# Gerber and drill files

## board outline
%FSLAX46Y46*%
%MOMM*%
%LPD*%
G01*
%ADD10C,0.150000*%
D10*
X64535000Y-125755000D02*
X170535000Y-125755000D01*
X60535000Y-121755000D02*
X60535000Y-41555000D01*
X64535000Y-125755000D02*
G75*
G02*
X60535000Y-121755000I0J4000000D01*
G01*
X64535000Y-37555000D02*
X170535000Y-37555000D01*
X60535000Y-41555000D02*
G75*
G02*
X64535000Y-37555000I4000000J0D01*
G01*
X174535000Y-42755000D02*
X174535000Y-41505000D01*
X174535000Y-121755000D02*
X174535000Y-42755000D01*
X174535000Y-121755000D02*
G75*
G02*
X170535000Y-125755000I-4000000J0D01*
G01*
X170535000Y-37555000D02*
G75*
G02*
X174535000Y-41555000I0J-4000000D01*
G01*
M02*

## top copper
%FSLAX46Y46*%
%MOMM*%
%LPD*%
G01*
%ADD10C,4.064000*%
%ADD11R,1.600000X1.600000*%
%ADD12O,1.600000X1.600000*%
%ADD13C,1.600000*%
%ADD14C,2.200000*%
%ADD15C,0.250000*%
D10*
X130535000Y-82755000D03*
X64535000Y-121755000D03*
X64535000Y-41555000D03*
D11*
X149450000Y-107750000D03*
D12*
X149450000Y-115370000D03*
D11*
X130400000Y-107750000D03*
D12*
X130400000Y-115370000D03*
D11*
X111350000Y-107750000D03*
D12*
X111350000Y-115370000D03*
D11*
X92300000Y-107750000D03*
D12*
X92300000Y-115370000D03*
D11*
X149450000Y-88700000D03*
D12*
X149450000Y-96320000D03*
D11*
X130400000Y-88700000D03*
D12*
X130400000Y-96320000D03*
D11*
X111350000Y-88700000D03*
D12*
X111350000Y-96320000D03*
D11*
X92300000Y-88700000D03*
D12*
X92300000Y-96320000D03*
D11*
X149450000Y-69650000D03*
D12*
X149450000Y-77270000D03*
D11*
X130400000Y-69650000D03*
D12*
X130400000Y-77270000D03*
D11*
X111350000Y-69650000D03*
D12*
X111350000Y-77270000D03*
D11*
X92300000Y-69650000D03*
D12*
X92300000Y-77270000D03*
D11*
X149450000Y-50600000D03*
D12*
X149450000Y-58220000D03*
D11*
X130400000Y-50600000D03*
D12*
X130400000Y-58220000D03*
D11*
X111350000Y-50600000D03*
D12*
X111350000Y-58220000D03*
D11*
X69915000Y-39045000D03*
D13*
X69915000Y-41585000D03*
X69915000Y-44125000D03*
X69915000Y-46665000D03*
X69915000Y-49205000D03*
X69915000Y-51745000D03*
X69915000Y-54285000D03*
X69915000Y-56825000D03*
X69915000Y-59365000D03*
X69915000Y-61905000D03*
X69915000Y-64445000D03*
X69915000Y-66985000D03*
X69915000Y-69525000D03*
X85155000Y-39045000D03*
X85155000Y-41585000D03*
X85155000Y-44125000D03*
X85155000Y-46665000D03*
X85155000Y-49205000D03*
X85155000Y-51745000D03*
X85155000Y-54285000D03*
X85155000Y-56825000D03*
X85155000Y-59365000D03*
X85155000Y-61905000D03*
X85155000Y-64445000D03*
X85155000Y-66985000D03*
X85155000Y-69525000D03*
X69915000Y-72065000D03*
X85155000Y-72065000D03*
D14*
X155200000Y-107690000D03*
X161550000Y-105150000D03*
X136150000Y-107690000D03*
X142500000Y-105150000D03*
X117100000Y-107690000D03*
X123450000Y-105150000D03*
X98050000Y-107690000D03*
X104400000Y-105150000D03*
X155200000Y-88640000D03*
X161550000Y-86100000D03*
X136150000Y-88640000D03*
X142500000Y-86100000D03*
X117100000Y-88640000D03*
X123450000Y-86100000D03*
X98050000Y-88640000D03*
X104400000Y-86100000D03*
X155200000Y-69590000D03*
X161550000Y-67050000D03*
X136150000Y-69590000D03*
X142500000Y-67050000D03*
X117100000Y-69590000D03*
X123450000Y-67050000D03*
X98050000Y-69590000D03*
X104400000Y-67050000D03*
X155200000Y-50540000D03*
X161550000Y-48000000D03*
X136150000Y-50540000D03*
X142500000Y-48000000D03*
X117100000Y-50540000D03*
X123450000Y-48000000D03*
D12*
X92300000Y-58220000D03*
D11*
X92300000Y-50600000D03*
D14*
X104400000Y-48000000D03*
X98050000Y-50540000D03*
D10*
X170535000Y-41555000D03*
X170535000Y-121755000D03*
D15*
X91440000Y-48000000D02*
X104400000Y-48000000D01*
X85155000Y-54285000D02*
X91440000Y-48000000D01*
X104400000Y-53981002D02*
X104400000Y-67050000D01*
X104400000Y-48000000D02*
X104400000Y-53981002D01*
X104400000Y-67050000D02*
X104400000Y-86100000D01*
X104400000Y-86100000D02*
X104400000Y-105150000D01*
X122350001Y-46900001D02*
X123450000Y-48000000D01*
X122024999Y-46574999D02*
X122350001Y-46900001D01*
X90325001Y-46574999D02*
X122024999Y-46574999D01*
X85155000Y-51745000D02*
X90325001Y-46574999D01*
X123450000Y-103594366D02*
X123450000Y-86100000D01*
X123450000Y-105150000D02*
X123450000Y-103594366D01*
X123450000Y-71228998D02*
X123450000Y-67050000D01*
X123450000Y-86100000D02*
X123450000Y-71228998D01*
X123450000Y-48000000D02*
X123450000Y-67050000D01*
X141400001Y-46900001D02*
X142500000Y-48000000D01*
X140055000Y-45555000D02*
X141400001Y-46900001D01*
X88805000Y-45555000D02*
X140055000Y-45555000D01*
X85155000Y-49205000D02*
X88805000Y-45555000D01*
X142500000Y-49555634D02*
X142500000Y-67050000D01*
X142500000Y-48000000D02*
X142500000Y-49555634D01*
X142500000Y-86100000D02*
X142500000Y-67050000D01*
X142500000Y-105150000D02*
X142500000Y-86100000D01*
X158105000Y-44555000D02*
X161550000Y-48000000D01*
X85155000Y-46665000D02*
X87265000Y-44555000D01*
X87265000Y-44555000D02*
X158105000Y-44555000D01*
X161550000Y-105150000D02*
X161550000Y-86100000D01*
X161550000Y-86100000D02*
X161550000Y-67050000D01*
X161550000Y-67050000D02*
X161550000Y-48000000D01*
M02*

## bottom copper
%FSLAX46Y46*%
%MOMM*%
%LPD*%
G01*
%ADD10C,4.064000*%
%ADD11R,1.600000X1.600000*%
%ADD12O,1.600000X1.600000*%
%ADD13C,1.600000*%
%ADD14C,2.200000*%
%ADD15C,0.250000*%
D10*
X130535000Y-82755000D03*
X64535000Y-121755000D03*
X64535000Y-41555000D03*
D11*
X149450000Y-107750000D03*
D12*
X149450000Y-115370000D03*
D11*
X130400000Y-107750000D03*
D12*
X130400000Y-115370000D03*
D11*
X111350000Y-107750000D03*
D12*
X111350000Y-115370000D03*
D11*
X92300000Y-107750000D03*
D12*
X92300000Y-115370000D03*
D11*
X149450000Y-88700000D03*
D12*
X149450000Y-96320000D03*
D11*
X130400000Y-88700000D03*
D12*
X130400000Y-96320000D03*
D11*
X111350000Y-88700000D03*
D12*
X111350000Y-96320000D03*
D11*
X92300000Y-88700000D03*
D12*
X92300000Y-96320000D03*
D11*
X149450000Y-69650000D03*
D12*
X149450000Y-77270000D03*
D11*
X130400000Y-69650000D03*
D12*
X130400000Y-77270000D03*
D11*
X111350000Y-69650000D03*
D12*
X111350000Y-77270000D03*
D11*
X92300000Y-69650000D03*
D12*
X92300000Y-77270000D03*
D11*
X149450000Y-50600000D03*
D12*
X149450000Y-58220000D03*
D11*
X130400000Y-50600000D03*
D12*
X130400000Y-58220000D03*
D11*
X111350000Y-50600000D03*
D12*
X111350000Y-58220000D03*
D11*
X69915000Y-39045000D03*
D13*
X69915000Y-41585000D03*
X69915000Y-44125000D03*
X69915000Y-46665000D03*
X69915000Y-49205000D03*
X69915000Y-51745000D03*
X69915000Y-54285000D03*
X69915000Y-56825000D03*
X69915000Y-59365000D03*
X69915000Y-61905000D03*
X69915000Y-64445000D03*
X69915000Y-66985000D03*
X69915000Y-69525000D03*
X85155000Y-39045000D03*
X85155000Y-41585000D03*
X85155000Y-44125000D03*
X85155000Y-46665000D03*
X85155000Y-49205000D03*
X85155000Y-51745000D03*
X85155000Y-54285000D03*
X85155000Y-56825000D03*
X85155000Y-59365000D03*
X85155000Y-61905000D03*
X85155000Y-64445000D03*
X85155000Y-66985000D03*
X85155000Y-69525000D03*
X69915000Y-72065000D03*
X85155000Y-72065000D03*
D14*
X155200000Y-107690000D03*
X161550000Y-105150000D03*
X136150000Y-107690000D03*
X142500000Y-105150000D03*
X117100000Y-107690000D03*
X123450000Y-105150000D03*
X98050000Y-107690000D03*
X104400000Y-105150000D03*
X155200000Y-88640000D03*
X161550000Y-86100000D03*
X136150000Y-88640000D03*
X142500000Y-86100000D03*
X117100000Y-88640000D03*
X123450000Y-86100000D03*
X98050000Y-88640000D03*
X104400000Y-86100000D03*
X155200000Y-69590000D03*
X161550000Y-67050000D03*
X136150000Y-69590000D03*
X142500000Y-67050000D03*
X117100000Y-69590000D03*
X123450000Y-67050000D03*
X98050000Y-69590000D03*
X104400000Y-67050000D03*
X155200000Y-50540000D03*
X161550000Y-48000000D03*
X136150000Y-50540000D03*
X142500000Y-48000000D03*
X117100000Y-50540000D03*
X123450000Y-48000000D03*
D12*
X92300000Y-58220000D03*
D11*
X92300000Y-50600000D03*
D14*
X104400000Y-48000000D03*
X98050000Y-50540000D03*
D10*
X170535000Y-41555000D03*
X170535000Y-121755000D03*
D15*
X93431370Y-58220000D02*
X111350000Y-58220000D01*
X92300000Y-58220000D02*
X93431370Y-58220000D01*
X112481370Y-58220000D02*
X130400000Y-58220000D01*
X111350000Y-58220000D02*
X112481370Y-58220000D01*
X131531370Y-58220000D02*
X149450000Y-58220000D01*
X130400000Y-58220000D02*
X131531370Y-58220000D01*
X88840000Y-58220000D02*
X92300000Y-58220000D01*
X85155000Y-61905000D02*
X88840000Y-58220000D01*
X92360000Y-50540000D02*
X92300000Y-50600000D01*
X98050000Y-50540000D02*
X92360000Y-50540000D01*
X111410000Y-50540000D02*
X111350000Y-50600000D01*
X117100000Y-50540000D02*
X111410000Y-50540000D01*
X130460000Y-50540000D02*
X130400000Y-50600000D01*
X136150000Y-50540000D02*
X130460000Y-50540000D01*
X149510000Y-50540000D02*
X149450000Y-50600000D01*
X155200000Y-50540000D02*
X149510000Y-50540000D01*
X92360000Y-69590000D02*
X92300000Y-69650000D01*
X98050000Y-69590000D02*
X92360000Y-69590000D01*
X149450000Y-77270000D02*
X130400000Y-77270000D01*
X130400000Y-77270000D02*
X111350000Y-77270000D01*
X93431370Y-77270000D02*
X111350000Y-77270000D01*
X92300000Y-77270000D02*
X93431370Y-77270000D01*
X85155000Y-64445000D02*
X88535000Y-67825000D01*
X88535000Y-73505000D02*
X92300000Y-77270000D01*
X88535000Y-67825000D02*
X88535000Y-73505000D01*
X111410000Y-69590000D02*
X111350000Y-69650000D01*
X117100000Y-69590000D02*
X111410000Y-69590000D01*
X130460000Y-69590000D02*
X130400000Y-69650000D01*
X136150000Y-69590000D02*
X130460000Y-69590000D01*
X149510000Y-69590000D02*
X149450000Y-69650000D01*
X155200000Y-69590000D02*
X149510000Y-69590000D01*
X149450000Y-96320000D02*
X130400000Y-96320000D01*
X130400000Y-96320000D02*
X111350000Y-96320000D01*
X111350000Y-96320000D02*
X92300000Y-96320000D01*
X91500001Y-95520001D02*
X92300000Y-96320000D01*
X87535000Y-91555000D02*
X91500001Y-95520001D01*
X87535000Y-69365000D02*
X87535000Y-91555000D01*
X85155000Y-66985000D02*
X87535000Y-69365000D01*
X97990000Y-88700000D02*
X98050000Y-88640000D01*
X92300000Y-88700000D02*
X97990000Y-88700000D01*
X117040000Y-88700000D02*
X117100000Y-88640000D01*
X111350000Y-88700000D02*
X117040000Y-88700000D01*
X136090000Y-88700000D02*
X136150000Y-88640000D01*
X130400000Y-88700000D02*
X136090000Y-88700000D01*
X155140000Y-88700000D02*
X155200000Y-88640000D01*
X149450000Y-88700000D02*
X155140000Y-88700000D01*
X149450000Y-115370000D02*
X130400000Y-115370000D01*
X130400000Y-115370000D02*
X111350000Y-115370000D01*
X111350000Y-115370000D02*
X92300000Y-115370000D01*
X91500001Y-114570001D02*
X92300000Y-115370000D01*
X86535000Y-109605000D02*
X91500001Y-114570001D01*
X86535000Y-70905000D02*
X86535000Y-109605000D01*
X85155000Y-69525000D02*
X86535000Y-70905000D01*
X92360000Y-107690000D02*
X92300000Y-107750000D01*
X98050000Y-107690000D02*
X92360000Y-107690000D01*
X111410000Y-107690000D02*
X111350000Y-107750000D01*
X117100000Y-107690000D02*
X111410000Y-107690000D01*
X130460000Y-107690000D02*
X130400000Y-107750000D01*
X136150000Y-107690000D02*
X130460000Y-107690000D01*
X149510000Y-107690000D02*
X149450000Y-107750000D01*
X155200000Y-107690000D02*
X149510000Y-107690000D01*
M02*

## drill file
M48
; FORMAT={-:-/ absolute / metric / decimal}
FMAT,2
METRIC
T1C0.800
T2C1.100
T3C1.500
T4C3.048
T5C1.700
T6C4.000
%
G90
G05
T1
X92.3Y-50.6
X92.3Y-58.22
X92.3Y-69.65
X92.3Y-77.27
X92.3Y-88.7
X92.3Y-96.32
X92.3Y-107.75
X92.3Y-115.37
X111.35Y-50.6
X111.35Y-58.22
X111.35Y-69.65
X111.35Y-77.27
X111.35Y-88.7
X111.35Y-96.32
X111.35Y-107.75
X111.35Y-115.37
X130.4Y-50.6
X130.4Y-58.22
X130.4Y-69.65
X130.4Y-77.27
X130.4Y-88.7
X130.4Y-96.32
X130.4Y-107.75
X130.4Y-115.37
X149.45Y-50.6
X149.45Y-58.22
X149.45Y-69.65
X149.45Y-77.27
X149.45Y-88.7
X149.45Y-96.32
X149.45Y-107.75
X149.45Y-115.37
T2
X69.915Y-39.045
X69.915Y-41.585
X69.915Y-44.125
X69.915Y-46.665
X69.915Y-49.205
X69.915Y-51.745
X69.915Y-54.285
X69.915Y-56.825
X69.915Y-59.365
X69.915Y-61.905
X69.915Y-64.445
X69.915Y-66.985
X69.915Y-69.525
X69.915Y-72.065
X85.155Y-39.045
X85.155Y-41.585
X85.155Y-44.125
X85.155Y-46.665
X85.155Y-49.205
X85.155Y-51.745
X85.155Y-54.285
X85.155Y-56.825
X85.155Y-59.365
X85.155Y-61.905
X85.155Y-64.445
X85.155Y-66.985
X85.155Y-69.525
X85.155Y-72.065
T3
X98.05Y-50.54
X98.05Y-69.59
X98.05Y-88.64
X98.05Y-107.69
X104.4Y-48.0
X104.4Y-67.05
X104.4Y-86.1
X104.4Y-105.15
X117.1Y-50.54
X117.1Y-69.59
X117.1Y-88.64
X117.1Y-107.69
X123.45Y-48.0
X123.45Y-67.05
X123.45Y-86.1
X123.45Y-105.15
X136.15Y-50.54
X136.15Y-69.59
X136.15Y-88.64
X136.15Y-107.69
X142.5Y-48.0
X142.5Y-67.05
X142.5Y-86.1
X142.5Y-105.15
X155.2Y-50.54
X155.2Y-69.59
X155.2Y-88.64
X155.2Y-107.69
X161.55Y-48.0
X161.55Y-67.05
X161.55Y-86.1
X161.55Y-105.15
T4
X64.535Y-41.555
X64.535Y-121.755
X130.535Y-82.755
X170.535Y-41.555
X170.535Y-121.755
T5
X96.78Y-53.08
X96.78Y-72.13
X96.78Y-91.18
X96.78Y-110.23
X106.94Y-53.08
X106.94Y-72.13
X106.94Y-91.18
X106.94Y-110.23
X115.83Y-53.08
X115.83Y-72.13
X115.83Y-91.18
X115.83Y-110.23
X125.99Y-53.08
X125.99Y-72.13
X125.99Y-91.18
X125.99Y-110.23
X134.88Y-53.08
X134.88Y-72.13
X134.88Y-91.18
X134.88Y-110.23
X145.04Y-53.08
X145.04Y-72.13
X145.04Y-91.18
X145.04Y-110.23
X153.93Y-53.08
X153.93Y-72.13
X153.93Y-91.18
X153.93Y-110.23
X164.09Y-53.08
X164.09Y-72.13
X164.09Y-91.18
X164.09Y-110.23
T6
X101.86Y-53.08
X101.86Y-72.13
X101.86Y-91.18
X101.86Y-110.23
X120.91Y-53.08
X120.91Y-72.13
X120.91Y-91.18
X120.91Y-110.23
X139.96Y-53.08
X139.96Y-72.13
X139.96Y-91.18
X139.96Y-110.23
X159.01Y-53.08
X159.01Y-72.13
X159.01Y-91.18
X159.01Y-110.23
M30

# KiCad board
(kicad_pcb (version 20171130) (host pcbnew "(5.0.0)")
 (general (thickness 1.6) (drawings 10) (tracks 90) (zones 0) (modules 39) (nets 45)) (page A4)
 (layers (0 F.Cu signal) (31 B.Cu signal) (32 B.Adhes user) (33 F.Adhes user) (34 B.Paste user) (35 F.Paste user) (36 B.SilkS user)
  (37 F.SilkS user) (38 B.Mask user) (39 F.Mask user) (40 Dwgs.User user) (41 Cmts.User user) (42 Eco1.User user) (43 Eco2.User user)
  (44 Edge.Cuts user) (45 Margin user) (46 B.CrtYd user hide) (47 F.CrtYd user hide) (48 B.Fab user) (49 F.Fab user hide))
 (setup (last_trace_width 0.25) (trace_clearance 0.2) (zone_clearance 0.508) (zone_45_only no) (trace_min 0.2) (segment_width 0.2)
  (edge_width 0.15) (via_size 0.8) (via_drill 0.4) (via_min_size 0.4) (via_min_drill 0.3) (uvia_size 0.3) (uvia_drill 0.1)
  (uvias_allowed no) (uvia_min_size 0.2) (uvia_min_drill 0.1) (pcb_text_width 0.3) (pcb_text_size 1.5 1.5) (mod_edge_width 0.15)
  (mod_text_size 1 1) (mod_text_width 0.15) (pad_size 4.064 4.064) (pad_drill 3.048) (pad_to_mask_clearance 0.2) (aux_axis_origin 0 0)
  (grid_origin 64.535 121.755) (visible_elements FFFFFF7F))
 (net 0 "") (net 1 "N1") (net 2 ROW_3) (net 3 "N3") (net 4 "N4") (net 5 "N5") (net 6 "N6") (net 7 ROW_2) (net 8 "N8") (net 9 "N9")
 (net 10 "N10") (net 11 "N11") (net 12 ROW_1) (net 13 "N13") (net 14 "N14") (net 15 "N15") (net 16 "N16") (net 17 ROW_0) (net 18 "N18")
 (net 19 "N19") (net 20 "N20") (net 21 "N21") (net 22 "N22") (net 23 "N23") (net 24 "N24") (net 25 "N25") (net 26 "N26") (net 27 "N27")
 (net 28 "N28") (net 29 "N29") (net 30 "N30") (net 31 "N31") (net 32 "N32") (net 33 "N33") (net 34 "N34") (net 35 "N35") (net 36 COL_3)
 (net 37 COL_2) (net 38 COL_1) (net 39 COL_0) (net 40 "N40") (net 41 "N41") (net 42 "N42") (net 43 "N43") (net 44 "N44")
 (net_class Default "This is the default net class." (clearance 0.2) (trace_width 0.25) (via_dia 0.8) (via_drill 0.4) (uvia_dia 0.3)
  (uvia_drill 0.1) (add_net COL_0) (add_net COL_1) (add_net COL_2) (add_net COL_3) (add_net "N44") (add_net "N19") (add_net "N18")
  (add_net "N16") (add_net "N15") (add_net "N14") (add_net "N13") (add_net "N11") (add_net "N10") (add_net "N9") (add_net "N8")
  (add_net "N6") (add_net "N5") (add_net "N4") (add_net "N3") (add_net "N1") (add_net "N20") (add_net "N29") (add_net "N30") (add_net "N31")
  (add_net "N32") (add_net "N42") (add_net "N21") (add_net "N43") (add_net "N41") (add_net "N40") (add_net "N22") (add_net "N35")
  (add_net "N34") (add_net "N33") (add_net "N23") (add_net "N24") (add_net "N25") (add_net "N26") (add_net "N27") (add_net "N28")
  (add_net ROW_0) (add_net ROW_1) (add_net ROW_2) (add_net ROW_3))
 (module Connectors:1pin (layer F.Cu) (at 130.535 82.755)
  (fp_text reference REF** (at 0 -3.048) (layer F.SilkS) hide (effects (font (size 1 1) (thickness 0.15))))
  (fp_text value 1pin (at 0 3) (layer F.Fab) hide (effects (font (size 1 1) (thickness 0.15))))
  (pad 1 thru_hole circle (at 0 0) (size 4.064 4.064) (drill 3.048) (layers *.Cu *.Mask)))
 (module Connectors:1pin (layer F.Cu) (at 64.535 121.755)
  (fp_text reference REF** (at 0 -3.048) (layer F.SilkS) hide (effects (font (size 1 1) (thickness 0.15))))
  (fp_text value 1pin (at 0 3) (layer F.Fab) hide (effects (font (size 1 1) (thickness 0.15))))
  (pad 1 thru_hole circle (at 0 0) (size 4.064 4.064) (drill 3.048) (layers *.Cu *.Mask)))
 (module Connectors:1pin (layer F.Cu) (at 64.535 41.555)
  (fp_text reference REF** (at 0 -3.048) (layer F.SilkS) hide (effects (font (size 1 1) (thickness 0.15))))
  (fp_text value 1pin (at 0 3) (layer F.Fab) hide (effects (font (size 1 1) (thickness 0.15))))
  (pad 1 thru_hole circle (at 0 0) (size 4.064 4.064) (drill 3.048) (layers *.Cu *.Mask)))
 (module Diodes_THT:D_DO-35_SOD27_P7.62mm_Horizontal (layer B.Cu) (at 149.45 107.75 270)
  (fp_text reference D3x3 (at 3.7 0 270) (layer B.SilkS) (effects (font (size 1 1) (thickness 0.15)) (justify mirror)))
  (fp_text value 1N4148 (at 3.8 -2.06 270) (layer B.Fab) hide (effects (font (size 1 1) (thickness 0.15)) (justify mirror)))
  (pad 1 thru_hole rect (at 0 0 270) (size 1.6 1.6) (drill 0.8) (layers *.Cu *.Mask) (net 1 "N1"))
  (pad 2 thru_hole oval (at 7.62 0 270) (size 1.6 1.6) (drill 0.8) (layers *.Cu *.Mask) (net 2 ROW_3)))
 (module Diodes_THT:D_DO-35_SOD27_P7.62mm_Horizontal (layer B.Cu) (at 130.4 107.75 270)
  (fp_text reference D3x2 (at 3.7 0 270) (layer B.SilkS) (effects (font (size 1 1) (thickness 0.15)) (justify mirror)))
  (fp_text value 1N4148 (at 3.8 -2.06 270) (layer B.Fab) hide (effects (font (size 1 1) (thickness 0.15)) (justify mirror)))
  (pad 1 thru_hole rect (at 0 0 270) (size 1.6 1.6) (drill 0.8) (layers *.Cu *.Mask) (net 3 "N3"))
  (pad 2 thru_hole oval (at 7.62 0 270) (size 1.6 1.6) (drill 0.8) (layers *.Cu *.Mask) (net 2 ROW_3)))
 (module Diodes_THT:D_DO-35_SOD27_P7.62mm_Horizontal (layer B.Cu) (at 111.35 107.75 270)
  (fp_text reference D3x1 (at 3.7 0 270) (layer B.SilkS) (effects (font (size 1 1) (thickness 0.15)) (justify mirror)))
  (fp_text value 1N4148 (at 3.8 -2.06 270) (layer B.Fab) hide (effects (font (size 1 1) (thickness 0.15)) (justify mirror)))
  (pad 1 thru_hole rect (at 0 0 270) (size 1.6 1.6) (drill 0.8) (layers *.Cu *.Mask) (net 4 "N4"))
  (pad 2 thru_hole oval (at 7.62 0 270) (size 1.6 1.6) (drill 0.8) (layers *.Cu *.Mask) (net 2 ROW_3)))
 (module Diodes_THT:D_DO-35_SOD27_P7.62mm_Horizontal (layer B.Cu) (at 92.3 107.75 270)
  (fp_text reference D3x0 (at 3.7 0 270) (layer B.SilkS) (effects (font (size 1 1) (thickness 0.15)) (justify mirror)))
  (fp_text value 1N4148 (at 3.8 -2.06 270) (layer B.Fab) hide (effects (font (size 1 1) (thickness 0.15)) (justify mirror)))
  (pad 1 thru_hole rect (at 0 0 270) (size 1.6 1.6) (drill 0.8) (layers *.Cu *.Mask) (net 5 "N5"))
  (pad 2 thru_hole oval (at 7.62 0 270) (size 1.6 1.6) (drill 0.8) (layers *.Cu *.Mask) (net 2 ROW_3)))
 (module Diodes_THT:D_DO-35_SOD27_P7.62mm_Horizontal (layer B.Cu) (at 149.45 88.7 270)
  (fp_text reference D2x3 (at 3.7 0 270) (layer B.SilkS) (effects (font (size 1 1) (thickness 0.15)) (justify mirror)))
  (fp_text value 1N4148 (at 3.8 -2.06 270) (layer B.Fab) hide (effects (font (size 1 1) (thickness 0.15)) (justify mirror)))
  (pad 1 thru_hole rect (at 0 0 270) (size 1.6 1.6) (drill 0.8) (layers *.Cu *.Mask) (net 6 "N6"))
  (pad 2 thru_hole oval (at 7.62 0 270) (size 1.6 1.6) (drill 0.8) (layers *.Cu *.Mask) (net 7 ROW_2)))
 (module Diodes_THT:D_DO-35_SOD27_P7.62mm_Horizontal (layer B.Cu) (at 130.4 88.7 270)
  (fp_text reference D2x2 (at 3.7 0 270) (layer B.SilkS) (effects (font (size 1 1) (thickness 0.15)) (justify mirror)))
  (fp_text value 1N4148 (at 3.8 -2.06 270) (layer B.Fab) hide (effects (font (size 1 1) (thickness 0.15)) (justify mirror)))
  (pad 1 thru_hole rect (at 0 0 270) (size 1.6 1.6) (drill 0.8) (layers *.Cu *.Mask) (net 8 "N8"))
  (pad 2 thru_hole oval (at 7.62 0 270) (size 1.6 1.6) (drill 0.8) (layers *.Cu *.Mask) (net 7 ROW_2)))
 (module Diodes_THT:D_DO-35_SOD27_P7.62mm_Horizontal (layer B.Cu) (at 111.35 88.7 270)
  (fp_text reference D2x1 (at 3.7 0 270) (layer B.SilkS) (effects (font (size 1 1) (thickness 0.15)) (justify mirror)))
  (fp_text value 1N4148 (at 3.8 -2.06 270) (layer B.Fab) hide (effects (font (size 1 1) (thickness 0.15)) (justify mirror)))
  (pad 1 thru_hole rect (at 0 0 270) (size 1.6 1.6) (drill 0.8) (layers *.Cu *.Mask) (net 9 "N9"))
  (pad 2 thru_hole oval (at 7.62 0 270) (size 1.6 1.6) (drill 0.8) (layers *.Cu *.Mask) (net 7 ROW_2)))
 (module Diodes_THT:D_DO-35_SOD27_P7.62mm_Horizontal (layer B.Cu) (at 92.3 88.7 270)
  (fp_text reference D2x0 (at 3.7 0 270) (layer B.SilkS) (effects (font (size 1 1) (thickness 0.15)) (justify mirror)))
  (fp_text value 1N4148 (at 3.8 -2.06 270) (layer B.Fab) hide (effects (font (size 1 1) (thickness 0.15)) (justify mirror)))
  (pad 1 thru_hole rect (at 0 0 270) (size 1.6 1.6) (drill 0.8) (layers *.Cu *.Mask) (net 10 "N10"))
  (pad 2 thru_hole oval (at 7.62 0 270) (size 1.6 1.6) (drill 0.8) (layers *.Cu *.Mask) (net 7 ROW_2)))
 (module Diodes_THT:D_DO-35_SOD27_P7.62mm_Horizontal (layer B.Cu) (at 149.45 69.65 270)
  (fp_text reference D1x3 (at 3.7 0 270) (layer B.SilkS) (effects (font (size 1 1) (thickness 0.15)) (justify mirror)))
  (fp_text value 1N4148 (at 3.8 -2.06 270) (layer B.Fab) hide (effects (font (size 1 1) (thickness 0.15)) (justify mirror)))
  (pad 1 thru_hole rect (at 0 0 270) (size 1.6 1.6) (drill 0.8) (layers *.Cu *.Mask) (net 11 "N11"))
  (pad 2 thru_hole oval (at 7.62 0 270) (size 1.6 1.6) (drill 0.8) (layers *.Cu *.Mask) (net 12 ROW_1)))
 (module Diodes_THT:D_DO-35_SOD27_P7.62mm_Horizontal (layer B.Cu) (at 130.4 69.65 270)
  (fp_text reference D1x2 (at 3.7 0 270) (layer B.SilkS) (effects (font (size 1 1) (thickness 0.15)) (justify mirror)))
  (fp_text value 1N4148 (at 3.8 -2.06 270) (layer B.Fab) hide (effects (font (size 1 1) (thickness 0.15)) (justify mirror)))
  (pad 1 thru_hole rect (at 0 0 270) (size 1.6 1.6) (drill 0.8) (layers *.Cu *.Mask) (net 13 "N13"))
  (pad 2 thru_hole oval (at 7.62 0 270) (size 1.6 1.6) (drill 0.8) (layers *.Cu *.Mask) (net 12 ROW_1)))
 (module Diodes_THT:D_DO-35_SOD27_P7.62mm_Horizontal (layer B.Cu) (at 111.35 69.65 270)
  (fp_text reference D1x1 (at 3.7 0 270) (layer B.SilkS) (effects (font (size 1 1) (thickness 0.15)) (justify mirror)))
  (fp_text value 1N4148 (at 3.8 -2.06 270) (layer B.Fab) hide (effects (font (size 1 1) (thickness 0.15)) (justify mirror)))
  (pad 1 thru_hole rect (at 0 0 270) (size 1.6 1.6) (drill 0.8) (layers *.Cu *.Mask) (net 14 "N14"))
  (pad 2 thru_hole oval (at 7.62 0 270) (size 1.6 1.6) (drill 0.8) (layers *.Cu *.Mask) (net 12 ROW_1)))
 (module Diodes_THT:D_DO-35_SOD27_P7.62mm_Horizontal (layer B.Cu) (at 92.3 69.65 270)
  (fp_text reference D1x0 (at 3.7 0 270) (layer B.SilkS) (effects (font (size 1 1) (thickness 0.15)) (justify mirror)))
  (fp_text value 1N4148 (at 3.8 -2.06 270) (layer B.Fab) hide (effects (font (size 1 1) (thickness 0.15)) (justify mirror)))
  (pad 1 thru_hole rect (at 0 0 270) (size 1.6 1.6) (drill 0.8) (layers *.Cu *.Mask) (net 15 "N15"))
  (pad 2 thru_hole oval (at 7.62 0 270) (size 1.6 1.6) (drill 0.8) (layers *.Cu *.Mask) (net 12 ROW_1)))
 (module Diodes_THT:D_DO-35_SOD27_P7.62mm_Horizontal (layer B.Cu) (at 149.45 50.6 270)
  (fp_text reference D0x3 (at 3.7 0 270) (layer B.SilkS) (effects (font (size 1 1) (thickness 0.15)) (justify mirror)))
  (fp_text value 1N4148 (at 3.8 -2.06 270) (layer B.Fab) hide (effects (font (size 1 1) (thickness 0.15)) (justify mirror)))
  (pad 1 thru_hole rect (at 0 0 270) (size 1.6 1.6) (drill 0.8) (layers *.Cu *.Mask) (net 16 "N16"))
  (pad 2 thru_hole oval (at 7.62 0 270) (size 1.6 1.6) (drill 0.8) (layers *.Cu *.Mask) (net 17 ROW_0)))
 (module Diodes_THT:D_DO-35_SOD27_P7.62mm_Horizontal (layer B.Cu) (at 130.4 50.6 270)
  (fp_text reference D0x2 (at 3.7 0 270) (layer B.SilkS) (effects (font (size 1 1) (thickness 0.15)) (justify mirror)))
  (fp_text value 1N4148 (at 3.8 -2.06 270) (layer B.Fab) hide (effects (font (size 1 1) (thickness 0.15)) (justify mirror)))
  (pad 1 thru_hole rect (at 0 0 270) (size 1.6 1.6) (drill 0.8) (layers *.Cu *.Mask) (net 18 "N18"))
  (pad 2 thru_hole oval (at 7.62 0 270) (size 1.6 1.6) (drill 0.8) (layers *.Cu *.Mask) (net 17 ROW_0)))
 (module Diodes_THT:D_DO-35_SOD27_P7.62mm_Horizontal (layer B.Cu) (at 111.35 50.6 270)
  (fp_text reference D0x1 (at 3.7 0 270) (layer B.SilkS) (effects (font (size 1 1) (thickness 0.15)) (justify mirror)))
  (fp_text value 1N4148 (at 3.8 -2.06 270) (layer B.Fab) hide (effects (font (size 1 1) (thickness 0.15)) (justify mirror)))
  (pad 1 thru_hole rect (at 0 0 270) (size 1.6 1.6) (drill 0.8) (layers *.Cu *.Mask) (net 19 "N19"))
  (pad 2 thru_hole oval (at 7.62 0 270) (size 1.6 1.6) (drill 0.8) (layers *.Cu *.Mask) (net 17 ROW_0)))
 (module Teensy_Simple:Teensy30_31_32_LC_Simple (layer F.Cu) (at 77.535 55.555 270)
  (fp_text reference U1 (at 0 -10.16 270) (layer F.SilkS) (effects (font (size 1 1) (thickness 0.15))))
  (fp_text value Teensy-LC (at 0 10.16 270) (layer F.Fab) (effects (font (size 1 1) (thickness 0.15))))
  (pad 1 thru_hole rect (at -16.51 7.62 270) (size 1.6 1.6) (drill 1.1) (layers *.Cu *.Mask F.SilkS) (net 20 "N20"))
  (pad 2 thru_hole circle (at -13.97 7.62 270) (size 1.6 1.6) (drill 1.1) (layers *.Cu *.Mask F.SilkS) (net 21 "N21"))
  (pad 3 thru_hole circle (at -11.43 7.62 270) (size 1.6 1.6) (drill 1.1) (layers *.Cu *.Mask F.SilkS) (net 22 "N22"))
  (pad 4 thru_hole circle (at -8.89 7.62 270) (size 1.6 1.6) (drill 1.1) (layers *.Cu *.Mask F.SilkS) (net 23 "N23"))
  (pad 5 thru_hole circle (at -6.35 7.62 270) (size 1.6 1.6) (drill 1.1) (layers *.Cu *.Mask F.SilkS) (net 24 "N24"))
  (pad 6 thru_hole circle (at -3.81 7.62 270) (size 1.6 1.6) (drill 1.1) (layers *.Cu *.Mask F.SilkS) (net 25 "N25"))
  (pad 7 thru_hole circle (at -1.27 7.62 270) (size 1.6 1.6) (drill 1.1) (layers *.Cu *.Mask F.SilkS) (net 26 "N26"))
  (pad 8 thru_hole circle (at 1.27 7.62 270) (size 1.6 1.6) (drill 1.1) (layers *.Cu *.Mask F.SilkS) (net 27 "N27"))
  (pad 9 thru_hole circle (at 3.81 7.62 270) (size 1.6 1.6) (drill 1.1) (layers *.Cu *.Mask F.SilkS) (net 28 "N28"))
  (pad 10 thru_hole circle (at 6.35 7.62 270) (size 1.6 1.6) (drill 1.1) (layers *.Cu *.Mask F.SilkS) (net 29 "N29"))
  (pad 11 thru_hole circle (at 8.89 7.62 270) (size 1.6 1.6) (drill 1.1) (layers *.Cu *.Mask F.SilkS) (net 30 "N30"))
  (pad 12 thru_hole circle (at 11.43 7.62 270) (size 1.6 1.6) (drill 1.1) (layers *.Cu *.Mask F.SilkS) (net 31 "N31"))
  (pad 13 thru_hole circle (at 13.97 7.62 270) (size 1.6 1.6) (drill 1.1) (layers *.Cu *.Mask F.SilkS) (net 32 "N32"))
  (pad 33 thru_hole circle (at -16.51 -7.62 270) (size 1.6 1.6) (drill 1.1) (layers *.Cu *.Mask F.SilkS) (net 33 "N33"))
  (pad 32 thru_hole circle (at -13.97 -7.62 270) (size 1.6 1.6) (drill 1.1) (layers *.Cu *.Mask F.SilkS) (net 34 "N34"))
  (pad 31 thru_hole circle (at -11.43 -7.62 270) (size 1.6 1.6) (drill 1.1) (layers *.Cu *.Mask F.SilkS) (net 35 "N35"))
  (pad 30 thru_hole circle (at -8.89 -7.62 270) (size 1.6 1.6) (drill 1.1) (layers *.Cu *.Mask F.SilkS) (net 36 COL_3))
  (pad 29 thru_hole circle (at -6.35 -7.62 270) (size 1.6 1.6) (drill 1.1) (layers *.Cu *.Mask F.SilkS) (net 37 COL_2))
  (pad 28 thru_hole circle (at -3.81 -7.62 270) (size 1.6 1.6) (drill 1.1) (layers *.Cu *.Mask F.SilkS) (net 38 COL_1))
  (pad 27 thru_hole circle (at -1.27 -7.62 270) (size 1.6 1.6) (drill 1.1) (layers *.Cu *.Mask F.SilkS) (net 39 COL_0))
  (pad 26 thru_hole circle (at 1.27 -7.62 270) (size 1.6 1.6) (drill 1.1) (layers *.Cu *.Mask F.SilkS) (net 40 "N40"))
  (pad 25 thru_hole circle (at 3.81 -7.62 270) (size 1.6 1.6) (drill 1.1) (layers *.Cu *.Mask F.SilkS) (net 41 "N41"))
  (pad 24 thru_hole circle (at 6.35 -7.62 270) (size 1.6 1.6) (drill 1.1) (layers *.Cu *.Mask F.SilkS) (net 17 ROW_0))
  (pad 23 thru_hole circle (at 8.89 -7.62 270) (size 1.6 1.6) (drill 1.1) (layers *.Cu *.Mask F.SilkS) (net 12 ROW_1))
  (pad 22 thru_hole circle (at 11.43 -7.62 270) (size 1.6 1.6) (drill 1.1) (layers *.Cu *.Mask F.SilkS) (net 7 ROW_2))
  (pad 21 thru_hole circle (at 13.97 -7.62 270) (size 1.6 1.6) (drill 1.1) (layers *.Cu *.Mask F.SilkS) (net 2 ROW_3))
  (pad 14 thru_hole circle (at 16.51 7.62 270) (size 1.6 1.6) (drill 1.1) (layers *.Cu *.Mask F.SilkS) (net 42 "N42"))
  (pad 20 thru_hole circle (at 16.51 -7.62 270) (size 1.6 1.6) (drill 1.1) (layers *.Cu *.Mask F.SilkS) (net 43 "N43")))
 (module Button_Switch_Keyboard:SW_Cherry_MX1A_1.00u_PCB (layer F.Cu) (at 161.55 105.15)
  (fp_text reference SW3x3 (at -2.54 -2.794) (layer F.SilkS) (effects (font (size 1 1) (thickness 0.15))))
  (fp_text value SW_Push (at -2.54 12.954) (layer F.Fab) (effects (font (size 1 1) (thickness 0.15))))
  (pad "" np_thru_hole circle (at 2.54 5.08) (size 1.7 1.7) (drill 1.7) (layers *.Cu *.Mask))
  (pad "" np_thru_hole circle (at -7.62 5.08) (size 1.7 1.7) (drill 1.7) (layers *.Cu *.Mask))
  (pad "" np_thru_hole circle (at -2.54 5.08) (size 4 4) (drill 4) (layers *.Cu *.Mask))
  (pad 2 thru_hole circle (at -6.35 2.54) (size 2.2 2.2) (drill 1.5) (layers *.Cu *.Mask) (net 1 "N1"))
  (pad 1 thru_hole circle (at 0 0) (size 2.2 2.2) (drill 1.5) (layers *.Cu *.Mask) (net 36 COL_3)))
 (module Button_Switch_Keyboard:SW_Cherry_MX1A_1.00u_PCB (layer F.Cu) (at 142.5 105.15)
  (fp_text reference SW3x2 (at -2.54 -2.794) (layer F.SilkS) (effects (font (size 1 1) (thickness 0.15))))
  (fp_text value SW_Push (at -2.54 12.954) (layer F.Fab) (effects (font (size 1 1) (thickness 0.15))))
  (pad "" np_thru_hole circle (at 2.54 5.08) (size 1.7 1.7) (drill 1.7) (layers *.Cu *.Mask))
  (pad "" np_thru_hole circle (at -7.62 5.08) (size 1.7 1.7) (drill 1.7) (layers *.Cu *.Mask))
  (pad "" np_thru_hole circle (at -2.54 5.08) (size 4 4) (drill 4) (layers *.Cu *.Mask))
  (pad 2 thru_hole circle (at -6.35 2.54) (size 2.2 2.2) (drill 1.5) (layers *.Cu *.Mask) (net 3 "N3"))
  (pad 1 thru_hole circle (at 0 0) (size 2.2 2.2) (drill 1.5) (layers *.Cu *.Mask) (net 37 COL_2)))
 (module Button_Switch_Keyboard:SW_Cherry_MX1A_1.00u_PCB (layer F.Cu) (at 123.45 105.15)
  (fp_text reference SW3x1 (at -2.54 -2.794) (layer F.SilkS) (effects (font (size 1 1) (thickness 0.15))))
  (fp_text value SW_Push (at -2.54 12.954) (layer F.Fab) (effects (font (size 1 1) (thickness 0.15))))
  (pad "" np_thru_hole circle (at 2.54 5.08) (size 1.7 1.7) (drill 1.7) (layers *.Cu *.Mask))
  (pad "" np_thru_hole circle (at -7.62 5.08) (size 1.7 1.7) (drill 1.7) (layers *.Cu *.Mask))
  (pad "" np_thru_hole circle (at -2.54 5.08) (size 4 4) (drill 4) (layers *.Cu *.Mask))
  (pad 2 thru_hole circle (at -6.35 2.54) (size 2.2 2.2) (drill 1.5) (layers *.Cu *.Mask) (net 4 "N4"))
  (pad 1 thru_hole circle (at 0 0) (size 2.2 2.2) (drill 1.5) (layers *.Cu *.Mask) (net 38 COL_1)))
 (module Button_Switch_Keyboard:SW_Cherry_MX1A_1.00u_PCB (layer F.Cu) (at 104.4 105.15)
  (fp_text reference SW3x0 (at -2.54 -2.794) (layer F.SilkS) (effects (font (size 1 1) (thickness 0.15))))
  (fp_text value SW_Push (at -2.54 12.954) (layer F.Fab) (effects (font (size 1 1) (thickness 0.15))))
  (pad "" np_thru_hole circle (at 2.54 5.08) (size 1.7 1.7) (drill 1.7) (layers *.Cu *.Mask))
  (pad "" np_thru_hole circle (at -7.62 5.08) (size 1.7 1.7) (drill 1.7) (layers *.Cu *.Mask))
  (pad "" np_thru_hole circle (at -2.54 5.08) (size 4 4) (drill 4) (layers *.Cu *.Mask))
  (pad 2 thru_hole circle (at -6.35 2.54) (size 2.2 2.2) (drill 1.5) (layers *.Cu *.Mask) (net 5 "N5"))
  (pad 1 thru_hole circle (at 0 0) (size 2.2 2.2) (drill 1.5) (layers *.Cu *.Mask) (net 39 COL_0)))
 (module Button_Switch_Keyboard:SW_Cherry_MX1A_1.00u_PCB (layer F.Cu) (at 161.55 86.1)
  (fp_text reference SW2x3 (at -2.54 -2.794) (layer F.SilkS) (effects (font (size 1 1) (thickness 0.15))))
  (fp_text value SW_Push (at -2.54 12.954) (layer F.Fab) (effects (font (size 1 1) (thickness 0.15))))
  (pad "" np_thru_hole circle (at 2.54 5.08) (size 1.7 1.7) (drill 1.7) (layers *.Cu *.Mask))
  (pad "" np_thru_hole circle (at -7.62 5.08) (size 1.7 1.7) (drill 1.7) (layers *.Cu *.Mask))
  (pad "" np_thru_hole circle (at -2.54 5.08) (size 4 4) (drill 4) (layers *.Cu *.Mask))
  (pad 2 thru_hole circle (at -6.35 2.54) (size 2.2 2.2) (drill 1.5) (layers *.Cu *.Mask) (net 6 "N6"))
  (pad 1 thru_hole circle (at 0 0) (size 2.2 2.2) (drill 1.5) (layers *.Cu *.Mask) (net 36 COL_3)))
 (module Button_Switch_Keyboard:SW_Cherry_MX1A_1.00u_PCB (layer F.Cu) (at 142.5 86.1)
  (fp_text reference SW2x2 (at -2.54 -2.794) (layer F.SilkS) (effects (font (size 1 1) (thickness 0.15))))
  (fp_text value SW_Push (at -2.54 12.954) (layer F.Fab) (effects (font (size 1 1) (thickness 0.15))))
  (pad "" np_thru_hole circle (at 2.54 5.08) (size 1.7 1.7) (drill 1.7) (layers *.Cu *.Mask))
  (pad "" np_thru_hole circle (at -7.62 5.08) (size 1.7 1.7) (drill 1.7) (layers *.Cu *.Mask))
  (pad "" np_thru_hole circle (at -2.54 5.08) (size 4 4) (drill 4) (layers *.Cu *.Mask))
  (pad 2 thru_hole circle (at -6.35 2.54) (size 2.2 2.2) (drill 1.5) (layers *.Cu *.Mask) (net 8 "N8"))
  (pad 1 thru_hole circle (at 0 0) (size 2.2 2.2) (drill 1.5) (layers *.Cu *.Mask) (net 37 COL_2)))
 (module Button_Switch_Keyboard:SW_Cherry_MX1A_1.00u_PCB (layer F.Cu) (at 123.45 86.1)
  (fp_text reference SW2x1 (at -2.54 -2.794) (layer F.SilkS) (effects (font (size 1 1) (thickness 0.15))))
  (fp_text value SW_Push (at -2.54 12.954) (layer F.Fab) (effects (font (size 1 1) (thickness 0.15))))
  (pad "" np_thru_hole circle (at 2.54 5.08) (size 1.7 1.7) (drill 1.7) (layers *.Cu *.Mask))
  (pad "" np_thru_hole circle (at -7.62 5.08) (size 1.7 1.7) (drill 1.7) (layers *.Cu *.Mask))
  (pad "" np_thru_hole circle (at -2.54 5.08) (size 4 4) (drill 4) (layers *.Cu *.Mask))
  (pad 2 thru_hole circle (at -6.35 2.54) (size 2.2 2.2) (drill 1.5) (layers *.Cu *.Mask) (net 9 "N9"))
  (pad 1 thru_hole circle (at 0 0) (size 2.2 2.2) (drill 1.5) (layers *.Cu *.Mask) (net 38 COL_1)))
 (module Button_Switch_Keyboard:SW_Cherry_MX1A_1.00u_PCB (layer F.Cu) (at 104.4 86.1)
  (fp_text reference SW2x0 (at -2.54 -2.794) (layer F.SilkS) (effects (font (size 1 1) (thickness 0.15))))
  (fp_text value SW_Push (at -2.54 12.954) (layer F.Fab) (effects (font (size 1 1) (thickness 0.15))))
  (pad "" np_thru_hole circle (at 2.54 5.08) (size 1.7 1.7) (drill 1.7) (layers *.Cu *.Mask))
  (pad "" np_thru_hole circle (at -7.62 5.08) (size 1.7 1.7) (drill 1.7) (layers *.Cu *.Mask))
  (pad "" np_thru_hole circle (at -2.54 5.08) (size 4 4) (drill 4) (layers *.Cu *.Mask))
  (pad 2 thru_hole circle (at -6.35 2.54) (size 2.2 2.2) (drill 1.5) (layers *.Cu *.Mask) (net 10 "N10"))
  (pad 1 thru_hole circle (at 0 0) (size 2.2 2.2) (drill 1.5) (layers *.Cu *.Mask) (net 39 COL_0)))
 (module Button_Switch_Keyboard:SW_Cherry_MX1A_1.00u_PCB (layer F.Cu) (at 161.55 67.05)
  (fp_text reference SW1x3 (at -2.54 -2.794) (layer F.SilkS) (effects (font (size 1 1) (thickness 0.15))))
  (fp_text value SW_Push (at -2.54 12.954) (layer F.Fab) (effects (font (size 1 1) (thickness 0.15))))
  (pad "" np_thru_hole circle (at 2.54 5.08) (size 1.7 1.7) (drill 1.7) (layers *.Cu *.Mask))
  (pad "" np_thru_hole circle (at -7.62 5.08) (size 1.7 1.7) (drill 1.7) (layers *.Cu *.Mask))
  (pad "" np_thru_hole circle (at -2.54 5.08) (size 4 4) (drill 4) (layers *.Cu *.Mask))
  (pad 2 thru_hole circle (at -6.35 2.54) (size 2.2 2.2) (drill 1.5) (layers *.Cu *.Mask) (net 11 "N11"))
  (pad 1 thru_hole circle (at 0 0) (size 2.2 2.2) (drill 1.5) (layers *.Cu *.Mask) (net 36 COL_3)))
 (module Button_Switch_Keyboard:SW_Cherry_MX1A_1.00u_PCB (layer F.Cu) (at 142.5 67.05)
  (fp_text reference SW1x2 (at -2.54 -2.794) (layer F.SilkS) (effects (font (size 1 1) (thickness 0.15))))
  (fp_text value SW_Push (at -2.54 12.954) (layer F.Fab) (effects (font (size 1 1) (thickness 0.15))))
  (pad "" np_thru_hole circle (at 2.54 5.08) (size 1.7 1.7) (drill 1.7) (layers *.Cu *.Mask))
  (pad "" np_thru_hole circle (at -7.62 5.08) (size 1.7 1.7) (drill 1.7) (layers *.Cu *.Mask))
  (pad "" np_thru_hole circle (at -2.54 5.08) (size 4 4) (drill 4) (layers *.Cu *.Mask))
  (pad 2 thru_hole circle (at -6.35 2.54) (size 2.2 2.2) (drill 1.5) (layers *.Cu *.Mask) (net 13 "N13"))
  (pad 1 thru_hole circle (at 0 0) (size 2.2 2.2) (drill 1.5) (layers *.Cu *.Mask) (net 37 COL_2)))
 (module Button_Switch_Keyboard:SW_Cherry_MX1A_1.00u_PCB (layer F.Cu) (at 123.45 67.05)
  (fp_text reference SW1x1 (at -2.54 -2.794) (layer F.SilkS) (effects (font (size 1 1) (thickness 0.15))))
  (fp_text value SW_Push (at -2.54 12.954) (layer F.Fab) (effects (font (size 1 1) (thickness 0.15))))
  (pad "" np_thru_hole circle (at 2.54 5.08) (size 1.7 1.7) (drill 1.7) (layers *.Cu *.Mask))
  (pad "" np_thru_hole circle (at -7.62 5.08) (size 1.7 1.7) (drill 1.7) (layers *.Cu *.Mask))
  (pad "" np_thru_hole circle (at -2.54 5.08) (size 4 4) (drill 4) (layers *.Cu *.Mask))
  (pad 2 thru_hole circle (at -6.35 2.54) (size 2.2 2.2) (drill 1.5) (layers *.Cu *.Mask) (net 14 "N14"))
  (pad 1 thru_hole circle (at 0 0) (size 2.2 2.2) (drill 1.5) (layers *.Cu *.Mask) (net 38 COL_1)))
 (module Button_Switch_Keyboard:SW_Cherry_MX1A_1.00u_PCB (layer F.Cu) (at 104.4 67.05)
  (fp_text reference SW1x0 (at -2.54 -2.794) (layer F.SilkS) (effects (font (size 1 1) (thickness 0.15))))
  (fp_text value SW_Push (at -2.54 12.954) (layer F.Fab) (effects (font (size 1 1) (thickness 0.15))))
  (pad "" np_thru_hole circle (at 2.54 5.08) (size 1.7 1.7) (drill 1.7) (layers *.Cu *.Mask))
  (pad "" np_thru_hole circle (at -7.62 5.08) (size 1.7 1.7) (drill 1.7) (layers *.Cu *.Mask))
  (pad "" np_thru_hole circle (at -2.54 5.08) (size 4 4) (drill 4) (layers *.Cu *.Mask))
  (pad 2 thru_hole circle (at -6.35 2.54) (size 2.2 2.2) (drill 1.5) (layers *.Cu *.Mask) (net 15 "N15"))
  (pad 1 thru_hole circle (at 0 0) (size 2.2 2.2) (drill 1.5) (layers *.Cu *.Mask) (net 39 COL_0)))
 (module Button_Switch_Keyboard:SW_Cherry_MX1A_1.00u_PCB (layer F.Cu) (at 161.55 48)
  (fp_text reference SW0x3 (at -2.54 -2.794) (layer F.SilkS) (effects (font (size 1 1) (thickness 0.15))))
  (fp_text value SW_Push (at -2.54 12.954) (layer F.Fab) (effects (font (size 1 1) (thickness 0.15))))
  (pad "" np_thru_hole circle (at 2.54 5.08) (size 1.7 1.7) (drill 1.7) (layers *.Cu *.Mask))
  (pad "" np_thru_hole circle (at -7.62 5.08) (size 1.7 1.7) (drill 1.7) (layers *.Cu *.Mask))
  (pad "" np_thru_hole circle (at -2.54 5.08) (size 4 4) (drill 4) (layers *.Cu *.Mask))
  (pad 2 thru_hole circle (at -6.35 2.54) (size 2.2 2.2) (drill 1.5) (layers *.Cu *.Mask) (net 16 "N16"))
  (pad 1 thru_hole circle (at 0 0) (size 2.2 2.2) (drill 1.5) (layers *.Cu *.Mask) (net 36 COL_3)))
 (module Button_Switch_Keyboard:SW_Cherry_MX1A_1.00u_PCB (layer F.Cu) (at 142.5 48)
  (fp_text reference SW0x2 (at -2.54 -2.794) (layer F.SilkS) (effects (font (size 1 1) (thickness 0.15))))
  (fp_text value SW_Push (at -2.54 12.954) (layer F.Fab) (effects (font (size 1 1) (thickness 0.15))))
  (pad "" np_thru_hole circle (at 2.54 5.08) (size 1.7 1.7) (drill 1.7) (layers *.Cu *.Mask))
  (pad "" np_thru_hole circle (at -7.62 5.08) (size 1.7 1.7) (drill 1.7) (layers *.Cu *.Mask))
  (pad "" np_thru_hole circle (at -2.54 5.08) (size 4 4) (drill 4) (layers *.Cu *.Mask))
  (pad 2 thru_hole circle (at -6.35 2.54) (size 2.2 2.2) (drill 1.5) (layers *.Cu *.Mask) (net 18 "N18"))
  (pad 1 thru_hole circle (at 0 0) (size 2.2 2.2) (drill 1.5) (layers *.Cu *.Mask) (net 37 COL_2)))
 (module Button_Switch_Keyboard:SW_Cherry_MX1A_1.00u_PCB (layer F.Cu) (at 123.45 48)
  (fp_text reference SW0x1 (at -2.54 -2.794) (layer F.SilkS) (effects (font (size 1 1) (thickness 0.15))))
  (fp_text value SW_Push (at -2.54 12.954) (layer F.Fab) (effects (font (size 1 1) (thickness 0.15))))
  (pad "" np_thru_hole circle (at 2.54 5.08) (size 1.7 1.7) (drill 1.7) (layers *.Cu *.Mask))
  (pad "" np_thru_hole circle (at -7.62 5.08) (size 1.7 1.7) (drill 1.7) (layers *.Cu *.Mask))
  (pad "" np_thru_hole circle (at -2.54 5.08) (size 4 4) (drill 4) (layers *.Cu *.Mask))
  (pad 2 thru_hole circle (at -6.35 2.54) (size 2.2 2.2) (drill 1.5) (layers *.Cu *.Mask) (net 19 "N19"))
  (pad 1 thru_hole circle (at 0 0) (size 2.2 2.2) (drill 1.5) (layers *.Cu *.Mask) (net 38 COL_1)))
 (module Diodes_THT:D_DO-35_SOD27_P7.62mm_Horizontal (layer B.Cu) (at 92.3 50.6 270)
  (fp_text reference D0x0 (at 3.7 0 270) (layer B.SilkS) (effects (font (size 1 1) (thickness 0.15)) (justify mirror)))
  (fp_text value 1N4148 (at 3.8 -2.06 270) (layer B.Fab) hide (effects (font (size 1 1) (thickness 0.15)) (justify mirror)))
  (pad 2 thru_hole oval (at 7.62 0 270) (size 1.6 1.6) (drill 0.8) (layers *.Cu *.Mask) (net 17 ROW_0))
  (pad 1 thru_hole rect (at 0 0 270) (size 1.6 1.6) (drill 0.8) (layers *.Cu *.Mask) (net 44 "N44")))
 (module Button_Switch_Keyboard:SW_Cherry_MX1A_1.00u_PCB (layer F.Cu) (at 104.4 48)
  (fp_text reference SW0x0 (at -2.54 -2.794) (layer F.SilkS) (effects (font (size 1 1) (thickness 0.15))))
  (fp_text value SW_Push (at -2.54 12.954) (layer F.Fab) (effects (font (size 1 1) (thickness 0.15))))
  (pad 1 thru_hole circle (at 0 0) (size 2.2 2.2) (drill 1.5) (layers *.Cu *.Mask) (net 39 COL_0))
  (pad 2 thru_hole circle (at -6.35 2.54) (size 2.2 2.2) (drill 1.5) (layers *.Cu *.Mask) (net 44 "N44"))
  (pad "" np_thru_hole circle (at -2.54 5.08) (size 4 4) (drill 4) (layers *.Cu *.Mask))
  (pad "" np_thru_hole circle (at -7.62 5.08) (size 1.7 1.7) (drill 1.7) (layers *.Cu *.Mask))
  (pad "" np_thru_hole circle (at 2.54 5.08) (size 1.7 1.7) (drill 1.7) (layers *.Cu *.Mask)))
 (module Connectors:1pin (layer F.Cu) (at 170.535 41.555)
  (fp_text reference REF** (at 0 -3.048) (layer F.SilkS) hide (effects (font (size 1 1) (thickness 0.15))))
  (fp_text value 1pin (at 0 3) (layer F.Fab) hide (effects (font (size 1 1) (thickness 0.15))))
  (pad 1 thru_hole circle (at 0 0) (size 4.064 4.064) (drill 3.048) (layers *.Cu *.Mask)))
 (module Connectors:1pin (layer F.Cu) (at 170.535 121.755)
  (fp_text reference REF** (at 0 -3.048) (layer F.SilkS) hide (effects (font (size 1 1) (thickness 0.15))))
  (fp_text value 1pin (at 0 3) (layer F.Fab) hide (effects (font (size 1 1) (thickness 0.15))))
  (pad 1 thru_hole circle (at 0 0) (size 4.064 4.064) (drill 3.048) (layers *.Cu *.Mask)))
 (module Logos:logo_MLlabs (layer F.Cu) (at 74.535 84.755)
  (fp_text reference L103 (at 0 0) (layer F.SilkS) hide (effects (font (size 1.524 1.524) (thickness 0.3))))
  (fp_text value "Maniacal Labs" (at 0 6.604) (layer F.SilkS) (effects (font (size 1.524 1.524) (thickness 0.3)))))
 (gr_line (start 64.535 125.755) (end 170.535 125.755) (layer Edge.Cuts) (width 0.15))
 (gr_line (start 60.535 121.755) (end 60.535 41.555) (layer Edge.Cuts) (width 0.15))
 (gr_arc (start 64.535 121.755) (end 60.535 121.755) (angle -90) (layer Edge.Cuts) (width 0.15))
 (gr_line (start 64.535 37.555) (end 170.535 37.555) (layer Edge.Cuts) (width 0.15))
 (gr_arc (start 64.535 41.555) (end 64.535 37.555) (angle -90) (layer Edge.Cuts) (width 0.15))
 (gr_line (start 174.535 42.755) (end 174.535 41.505) (layer Edge.Cuts) (width 0.15))
 (gr_line (start 174.535 121.755) (end 174.535 42.755) (layer Edge.Cuts) (width 0.15))
 (gr_arc (start 170.535 121.755) (end 170.535 125.755) (angle -90) (layer Edge.Cuts) (width 0.15))
 (gr_arc (start 170.535 41.555) (end 174.535 41.555) (angle -90) (layer Edge.Cuts) (width 0.15))
 (segment (start 93.43137 58.22) (end 111.35 58.22) (width 0.25) (layer B.Cu) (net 17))
 (segment (start 92.3 58.22) (end 93.43137 58.22) (width 0.25) (layer B.Cu) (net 17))
 (segment (start 112.48137 58.22) (end 130.4 58.22) (width 0.25) (layer B.Cu) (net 17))
 (segment (start 111.35 58.22) (end 112.48137 58.22) (width 0.25) (layer B.Cu) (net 17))
 (segment (start 131.53137 58.22) (end 149.45 58.22) (width 0.25) (layer B.Cu) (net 17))
 (segment (start 130.4 58.22) (end 131.53137 58.22) (width 0.25) (layer B.Cu) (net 17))
 (segment (start 88.84 58.22) (end 92.3 58.22) (width 0.25) (layer B.Cu) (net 17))
 (segment (start 85.155 61.905) (end 88.84 58.22) (width 0.25) (layer B.Cu) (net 17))
 (segment (start 92.36 50.54) (end 92.3 50.6) (width 0.25) (layer B.Cu) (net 44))
 (segment (start 98.05 50.54) (end 92.36 50.54) (width 0.25) (layer B.Cu) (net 44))
 (segment (start 111.41 50.54) (end 111.35 50.6) (width 0.25) (layer B.Cu) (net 19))
 (segment (start 117.1 50.54) (end 111.41 50.54) (width 0.25) (layer B.Cu) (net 19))
 (segment (start 130.46 50.54) (end 130.4 50.6) (width 0.25) (layer B.Cu) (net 18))
 (segment (start 136.15 50.54) (end 130.46 50.54) (width 0.25) (layer B.Cu) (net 18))
 (segment (start 149.51 50.54) (end 149.45 50.6) (width 0.25) (layer B.Cu) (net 16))
 (segment (start 155.2 50.54) (end 149.51 50.54) (width 0.25) (layer B.Cu) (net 16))
 (segment (start 92.36 69.59) (end 92.3 69.65) (width 0.25) (layer B.Cu) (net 15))
 (segment (start 98.05 69.59) (end 92.36 69.59) (width 0.25) (layer B.Cu) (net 15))
 (segment (start 149.45 77.27) (end 130.4 77.27) (width 0.25) (layer B.Cu) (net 12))
 (segment (start 130.4 77.27) (end 111.35 77.27) (width 0.25) (layer B.Cu) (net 12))
 (segment (start 93.43137 77.27) (end 111.35 77.27) (width 0.25) (layer B.Cu) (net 12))
 (segment (start 92.3 77.27) (end 93.43137 77.27) (width 0.25) (layer B.Cu) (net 12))
 (segment (start 85.155 64.445) (end 88.535 67.825) (width 0.25) (layer B.Cu) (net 12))
 (segment (start 88.535 73.505) (end 92.3 77.27) (width 0.25) (layer B.Cu) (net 12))
 (segment (start 88.535 67.825) (end 88.535 73.505) (width 0.25) (layer B.Cu) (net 12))
 (segment (start 111.41 69.59) (end 111.35 69.65) (width 0.25) (layer B.Cu) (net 14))
 (segment (start 117.1 69.59) (end 111.41 69.59) (width 0.25) (layer B.Cu) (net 14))
 (segment (start 130.46 69.59) (end 130.4 69.65) (width 0.25) (layer B.Cu) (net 13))
 (segment (start 136.15 69.59) (end 130.46 69.59) (width 0.25) (layer B.Cu) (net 13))
 (segment (start 149.51 69.59) (end 149.45 69.65) (width 0.25) (layer B.Cu) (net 11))
 (segment (start 155.2 69.59) (end 149.51 69.59) (width 0.25) (layer B.Cu) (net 11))
 (segment (start 149.45 96.32) (end 130.4 96.32) (width 0.25) (layer B.Cu) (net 7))
 (segment (start 130.4 96.32) (end 111.35 96.32) (width 0.25) (layer B.Cu) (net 7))
 (segment (start 111.35 96.32) (end 92.3 96.32) (width 0.25) (layer B.Cu) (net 7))
 (segment (start 91.500001 95.520001) (end 92.3 96.32) (width 0.25) (layer B.Cu) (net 7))
 (segment (start 87.535 91.555) (end 91.500001 95.520001) (width 0.25) (layer B.Cu) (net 7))
 (segment (start 87.535 69.365) (end 87.535 91.555) (width 0.25) (layer B.Cu) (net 7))
 (segment (start 85.155 66.985) (end 87.535 69.365) (width 0.25) (layer B.Cu) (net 7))
 (segment (start 97.99 88.7) (end 98.05 88.64) (width 0.25) (layer B.Cu) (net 10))
 (segment (start 92.3 88.7) (end 97.99 88.7) (width 0.25) (layer B.Cu) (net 10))
 (segment (start 117.04 88.7) (end 117.1 88.64) (width 0.25) (layer B.Cu) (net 9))
 (segment (start 111.35 88.7) (end 117.04 88.7) (width 0.25) (layer B.Cu) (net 9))
 (segment (start 136.09 88.7) (end 136.15 88.64) (width 0.25) (layer B.Cu) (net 8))
 (segment (start 130.4 88.7) (end 136.09 88.7) (width 0.25) (layer B.Cu) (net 8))
 (segment (start 155.14 88.7) (end 155.2 88.64) (width 0.25) (layer B.Cu) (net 6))
 (segment (start 149.45 88.7) (end 155.14 88.7) (width 0.25) (layer B.Cu) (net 6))
 (segment (start 149.45 115.37) (end 130.4 115.37) (width 0.25) (layer B.Cu) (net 2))
 (segment (start 130.4 115.37) (end 111.35 115.37) (width 0.25) (layer B.Cu) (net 2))
 (segment (start 111.35 115.37) (end 92.3 115.37) (width 0.25) (layer B.Cu) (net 2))
 (segment (start 91.500001 114.570001) (end 92.3 115.37) (width 0.25) (layer B.Cu) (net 2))
 (segment (start 86.535 109.605) (end 91.500001 114.570001) (width 0.25) (layer B.Cu) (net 2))
 (segment (start 86.535 70.905) (end 86.535 109.605) (width 0.25) (layer B.Cu) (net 2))
 (segment (start 85.155 69.525) (end 86.535 70.905) (width 0.25) (layer B.Cu) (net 2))
 (segment (start 92.36 107.69) (end 92.3 107.75) (width 0.25) (layer B.Cu) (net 5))
 (segment (start 98.05 107.69) (end 92.36 107.69) (width 0.25) (layer B.Cu) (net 5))
 (segment (start 111.41 107.69) (end 111.35 107.75) (width 0.25) (layer B.Cu) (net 4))
 (segment (start 117.1 107.69) (end 111.41 107.69) (width 0.25) (layer B.Cu) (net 4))
 (segment (start 130.46 107.69) (end 130.4 107.75) (width 0.25) (layer B.Cu) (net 3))
 (segment (start 136.15 107.69) (end 130.46 107.69) (width 0.25) (layer B.Cu) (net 3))
 (segment (start 149.51 107.69) (end 149.45 107.75) (width 0.25) (layer B.Cu) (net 1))
 (segment (start 155.2 107.69) (end 149.51 107.69) (width 0.25) (layer B.Cu) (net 1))
 (segment (start 91.44 48) (end 104.4 48) (width 0.25) (layer F.Cu) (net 39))
 (segment (start 85.155 54.285) (end 91.44 48) (width 0.25) (layer F.Cu) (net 39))
 (segment (start 104.4 53.981002) (end 104.4 67.05) (width 0.25) (layer F.Cu) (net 39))
 (segment (start 104.4 48) (end 104.4 53.981002) (width 0.25) (layer F.Cu) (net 39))
 (segment (start 104.4 67.05) (end 104.4 86.1) (width 0.25) (layer F.Cu) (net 39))
 (segment (start 104.4 86.1) (end 104.4 105.15) (width 0.25) (layer F.Cu) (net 39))
 (segment (start 122.350001 46.900001) (end 123.45 48) (width 0.25) (layer F.Cu) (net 38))
 (segment (start 122.024999 46.574999) (end 122.350001 46.900001) (width 0.25) (layer F.Cu) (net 38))
 (segment (start 90.325001 46.574999) (end 122.024999 46.574999) (width 0.25) (layer F.Cu) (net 38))
 (segment (start 85.155 51.745) (end 90.325001 46.574999) (width 0.25) (layer F.Cu) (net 38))
 (segment (start 123.45 103.594366) (end 123.45 86.1) (width 0.25) (layer F.Cu) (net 38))
 (segment (start 123.45 105.15) (end 123.45 103.594366) (width 0.25) (layer F.Cu) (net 38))
 (segment (start 123.45 71.228998) (end 123.45 67.05) (width 0.25) (layer F.Cu) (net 38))
 (segment (start 123.45 86.1) (end 123.45 71.228998) (width 0.25) (layer F.Cu) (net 38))
 (segment (start 123.45 48) (end 123.45 67.05) (width 0.25) (layer F.Cu) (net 38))
 (segment (start 141.400001 46.900001) (end 142.5 48) (width 0.25) (layer F.Cu) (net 37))
 (segment (start 140.055 45.555) (end 141.400001 46.900001) (width 0.25) (layer F.Cu) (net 37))
 (segment (start 88.805 45.555) (end 140.055 45.555) (width 0.25) (layer F.Cu) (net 37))
 (segment (start 85.155 49.205) (end 88.805 45.555) (width 0.25) (layer F.Cu) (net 37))
 (segment (start 142.5 49.555634) (end 142.5 67.05) (width 0.25) (layer F.Cu) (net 37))
 (segment (start 142.5 48) (end 142.5 49.555634) (width 0.25) (layer F.Cu) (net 37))
 (segment (start 142.5 86.1) (end 142.5 67.05) (width 0.25) (layer F.Cu) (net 37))
 (segment (start 142.5 105.15) (end 142.5 86.1) (width 0.25) (layer F.Cu) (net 37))
 (segment (start 158.105 44.555) (end 161.55 48) (width 0.25) (layer F.Cu) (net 36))
 (segment (start 85.155 46.665) (end 87.265 44.555) (width 0.25) (layer F.Cu) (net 36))
 (segment (start 87.265 44.555) (end 158.105 44.555) (width 0.25) (layer F.Cu) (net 36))
 (segment (start 161.55 105.15) (end 161.55 86.1) (width 0.25) (layer F.Cu) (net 36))
 (segment (start 161.55 86.1) (end 161.55 67.05) (width 0.25) (layer F.Cu) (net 36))
 (segment (start 161.55 67.05) (end 161.55 48) (width 0.25) (layer F.Cu) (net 36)))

